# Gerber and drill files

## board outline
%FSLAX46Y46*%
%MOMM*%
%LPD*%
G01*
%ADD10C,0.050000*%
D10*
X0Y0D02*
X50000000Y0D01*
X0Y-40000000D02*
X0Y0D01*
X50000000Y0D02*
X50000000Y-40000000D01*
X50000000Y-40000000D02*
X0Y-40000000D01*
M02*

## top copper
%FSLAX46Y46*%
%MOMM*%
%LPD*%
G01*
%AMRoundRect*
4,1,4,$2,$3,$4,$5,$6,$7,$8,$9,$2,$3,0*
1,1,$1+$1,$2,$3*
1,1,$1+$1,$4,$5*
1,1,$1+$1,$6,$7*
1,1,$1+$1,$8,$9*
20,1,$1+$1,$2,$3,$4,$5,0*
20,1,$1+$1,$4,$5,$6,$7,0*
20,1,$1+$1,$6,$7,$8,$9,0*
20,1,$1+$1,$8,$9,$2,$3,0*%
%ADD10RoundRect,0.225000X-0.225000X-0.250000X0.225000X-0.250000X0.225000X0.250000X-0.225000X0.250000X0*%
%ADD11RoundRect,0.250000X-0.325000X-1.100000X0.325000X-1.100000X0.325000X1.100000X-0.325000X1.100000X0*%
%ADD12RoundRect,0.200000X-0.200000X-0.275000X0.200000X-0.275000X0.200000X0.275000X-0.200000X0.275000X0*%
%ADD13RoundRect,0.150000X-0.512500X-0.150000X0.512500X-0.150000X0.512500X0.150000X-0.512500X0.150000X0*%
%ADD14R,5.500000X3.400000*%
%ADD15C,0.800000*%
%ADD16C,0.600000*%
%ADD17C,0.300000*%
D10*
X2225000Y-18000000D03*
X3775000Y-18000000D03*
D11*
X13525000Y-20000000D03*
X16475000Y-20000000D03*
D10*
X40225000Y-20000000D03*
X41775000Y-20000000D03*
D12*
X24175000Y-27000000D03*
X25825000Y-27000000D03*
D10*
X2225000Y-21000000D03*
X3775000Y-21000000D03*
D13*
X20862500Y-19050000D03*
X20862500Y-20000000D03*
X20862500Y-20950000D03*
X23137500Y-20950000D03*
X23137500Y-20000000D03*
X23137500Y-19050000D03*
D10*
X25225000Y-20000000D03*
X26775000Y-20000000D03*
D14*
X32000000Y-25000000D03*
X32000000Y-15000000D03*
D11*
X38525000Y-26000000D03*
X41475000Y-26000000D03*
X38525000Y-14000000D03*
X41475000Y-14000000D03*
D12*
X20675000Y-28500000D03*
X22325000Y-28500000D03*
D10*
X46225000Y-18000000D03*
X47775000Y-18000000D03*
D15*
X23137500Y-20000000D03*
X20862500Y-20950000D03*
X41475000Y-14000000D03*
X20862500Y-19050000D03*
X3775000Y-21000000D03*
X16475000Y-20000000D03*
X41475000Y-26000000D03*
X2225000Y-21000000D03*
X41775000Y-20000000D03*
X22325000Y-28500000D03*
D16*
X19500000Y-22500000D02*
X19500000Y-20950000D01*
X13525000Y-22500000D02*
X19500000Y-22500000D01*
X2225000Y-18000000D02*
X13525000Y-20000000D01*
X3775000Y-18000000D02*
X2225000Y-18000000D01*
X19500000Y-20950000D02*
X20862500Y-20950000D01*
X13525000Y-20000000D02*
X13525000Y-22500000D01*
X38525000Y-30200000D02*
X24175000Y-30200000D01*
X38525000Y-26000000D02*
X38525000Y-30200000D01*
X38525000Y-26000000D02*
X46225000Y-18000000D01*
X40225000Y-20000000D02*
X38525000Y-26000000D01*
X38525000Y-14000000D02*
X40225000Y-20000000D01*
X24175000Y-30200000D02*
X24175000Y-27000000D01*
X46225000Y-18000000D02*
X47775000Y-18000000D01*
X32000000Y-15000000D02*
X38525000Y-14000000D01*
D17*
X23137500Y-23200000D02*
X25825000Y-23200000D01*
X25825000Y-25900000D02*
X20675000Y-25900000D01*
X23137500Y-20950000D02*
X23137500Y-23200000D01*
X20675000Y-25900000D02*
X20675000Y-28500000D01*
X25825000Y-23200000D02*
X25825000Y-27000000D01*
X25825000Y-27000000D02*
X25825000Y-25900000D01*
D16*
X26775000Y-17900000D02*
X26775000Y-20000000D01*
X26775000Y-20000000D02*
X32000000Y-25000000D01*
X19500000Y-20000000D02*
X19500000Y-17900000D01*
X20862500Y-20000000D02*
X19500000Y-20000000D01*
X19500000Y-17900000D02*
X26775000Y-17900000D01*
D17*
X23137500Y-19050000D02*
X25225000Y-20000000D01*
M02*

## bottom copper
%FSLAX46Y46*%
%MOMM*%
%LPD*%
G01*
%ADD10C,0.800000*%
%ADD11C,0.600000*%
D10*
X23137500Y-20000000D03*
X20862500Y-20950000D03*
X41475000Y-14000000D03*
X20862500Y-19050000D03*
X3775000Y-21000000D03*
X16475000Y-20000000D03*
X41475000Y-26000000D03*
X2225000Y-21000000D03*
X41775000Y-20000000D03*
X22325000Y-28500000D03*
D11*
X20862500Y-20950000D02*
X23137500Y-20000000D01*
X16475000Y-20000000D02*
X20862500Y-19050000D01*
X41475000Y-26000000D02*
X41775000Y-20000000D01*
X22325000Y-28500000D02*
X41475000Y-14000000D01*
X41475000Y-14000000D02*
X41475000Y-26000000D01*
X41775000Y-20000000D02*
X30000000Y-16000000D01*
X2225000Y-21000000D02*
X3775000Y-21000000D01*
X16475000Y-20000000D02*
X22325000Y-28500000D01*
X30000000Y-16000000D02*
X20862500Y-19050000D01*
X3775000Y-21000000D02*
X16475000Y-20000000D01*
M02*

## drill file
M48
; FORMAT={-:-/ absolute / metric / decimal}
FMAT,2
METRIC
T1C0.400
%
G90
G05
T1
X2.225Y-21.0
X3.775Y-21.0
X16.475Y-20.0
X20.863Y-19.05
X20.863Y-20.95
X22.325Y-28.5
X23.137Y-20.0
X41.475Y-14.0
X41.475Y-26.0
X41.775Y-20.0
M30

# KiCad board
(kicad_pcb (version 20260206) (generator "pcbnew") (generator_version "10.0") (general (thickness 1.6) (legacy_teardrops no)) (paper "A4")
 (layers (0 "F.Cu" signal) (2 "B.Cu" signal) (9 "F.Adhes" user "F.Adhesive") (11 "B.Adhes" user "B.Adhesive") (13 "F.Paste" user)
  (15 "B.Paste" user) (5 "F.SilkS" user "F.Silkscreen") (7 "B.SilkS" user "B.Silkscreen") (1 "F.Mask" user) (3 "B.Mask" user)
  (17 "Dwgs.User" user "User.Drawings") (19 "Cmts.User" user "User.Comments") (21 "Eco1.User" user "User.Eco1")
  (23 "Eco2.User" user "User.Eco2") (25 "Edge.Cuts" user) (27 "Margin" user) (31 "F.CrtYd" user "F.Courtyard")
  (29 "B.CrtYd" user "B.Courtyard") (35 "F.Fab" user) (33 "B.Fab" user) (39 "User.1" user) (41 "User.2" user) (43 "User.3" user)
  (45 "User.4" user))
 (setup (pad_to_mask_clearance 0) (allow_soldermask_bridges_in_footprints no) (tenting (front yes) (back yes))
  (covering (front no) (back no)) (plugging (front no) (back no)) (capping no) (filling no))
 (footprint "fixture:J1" (layer "F.Cu") (at 3 18)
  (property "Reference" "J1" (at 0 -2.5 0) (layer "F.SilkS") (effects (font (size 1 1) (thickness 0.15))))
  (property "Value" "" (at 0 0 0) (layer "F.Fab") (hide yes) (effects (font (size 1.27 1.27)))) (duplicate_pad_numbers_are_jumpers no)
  (pad "1" smd roundrect (at -0.775 0) (size 0.9 0.95) (layers "F.Cu" "F.Mask" "F.Paste") (roundrect_rratio 0.25) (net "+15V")
   (thermal_bridge_angle 45))
  (pad "2" smd roundrect (at 0.775 0) (size 0.9 0.95) (layers "F.Cu" "F.Mask" "F.Paste") (roundrect_rratio 0.25) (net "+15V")
   (thermal_bridge_angle 45)))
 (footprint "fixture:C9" (layer "F.Cu") (at 15 20)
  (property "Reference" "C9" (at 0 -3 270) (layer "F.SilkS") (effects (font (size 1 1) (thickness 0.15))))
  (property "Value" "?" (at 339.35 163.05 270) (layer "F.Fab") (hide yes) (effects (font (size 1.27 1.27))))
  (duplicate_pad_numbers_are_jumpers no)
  (pad "1" smd roundrect (at -1.475 0) (size 1.15 2.7) (layers "F.Cu" "F.Mask" "F.Paste") (roundrect_rratio 0.217391) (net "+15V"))
  (pad "2" smd roundrect (at 1.475 0) (size 1.15 2.7) (layers "F.Cu" "F.Mask" "F.Paste") (roundrect_rratio 0.217391) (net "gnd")))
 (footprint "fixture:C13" (layer "F.Cu") (at 41 20)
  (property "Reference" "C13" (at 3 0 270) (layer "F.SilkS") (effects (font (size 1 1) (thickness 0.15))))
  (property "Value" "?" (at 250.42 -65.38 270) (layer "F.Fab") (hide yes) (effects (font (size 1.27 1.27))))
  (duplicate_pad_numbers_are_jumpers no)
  (pad "1" smd roundrect (at -0.775 0) (size 0.9 0.95) (layers "F.Cu" "F.Mask" "F.Paste") (roundrect_rratio 0.25) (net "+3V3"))
  (pad "2" smd roundrect (at 0.775 0) (size 0.9 0.95) (layers "F.Cu" "F.Mask" "F.Paste") (roundrect_rratio 0.25) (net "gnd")))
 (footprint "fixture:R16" (layer "F.Cu") (at 25 27)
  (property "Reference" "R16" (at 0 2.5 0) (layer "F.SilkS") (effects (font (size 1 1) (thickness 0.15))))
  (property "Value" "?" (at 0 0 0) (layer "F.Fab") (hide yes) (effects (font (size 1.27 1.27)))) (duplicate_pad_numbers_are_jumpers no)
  (pad "1" smd roundrect (at -0.825 0) (size 0.8 0.95) (layers "F.Cu" "F.Mask" "F.Paste") (roundrect_rratio 0.25) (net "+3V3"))
  (pad "2" smd roundrect (at 0.825 0) (size 0.8 0.95) (layers "F.Cu" "F.Mask" "F.Paste") (roundrect_rratio 0.25) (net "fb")))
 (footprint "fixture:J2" (layer "F.Cu") (at 3 21)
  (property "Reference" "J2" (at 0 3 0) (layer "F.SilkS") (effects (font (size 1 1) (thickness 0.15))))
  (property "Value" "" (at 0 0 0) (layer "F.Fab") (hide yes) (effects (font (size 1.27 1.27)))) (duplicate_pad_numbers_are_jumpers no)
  (pad "1" smd roundrect (at -0.775 0) (size 0.9 0.95) (layers "F.Cu" "F.Mask" "F.Paste") (roundrect_rratio 0.25) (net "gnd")
   (thermal_bridge_angle 45))
  (pad "2" smd roundrect (at 0.775 0) (size 0.9 0.95) (layers "F.Cu" "F.Mask" "F.Paste") (roundrect_rratio 0.25) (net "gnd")
   (thermal_bridge_angle 45)))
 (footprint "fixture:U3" (layer "F.Cu") (at 22 20)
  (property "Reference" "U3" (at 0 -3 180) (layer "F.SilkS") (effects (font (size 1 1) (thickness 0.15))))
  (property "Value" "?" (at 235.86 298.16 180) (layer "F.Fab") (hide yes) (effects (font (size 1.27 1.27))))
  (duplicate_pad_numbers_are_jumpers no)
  (pad "1" smd roundrect (at -1.1375 -0.95) (size 1.325 0.6) (layers "F.Cu" "F.Mask" "F.Paste") (roundrect_rratio 0.25) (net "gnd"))
  (pad "2" smd roundrect (at -1.1375 0) (size 1.325 0.6) (layers "F.Cu" "F.Mask" "F.Paste") (roundrect_rratio 0.25) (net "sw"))
  (pad "3" smd roundrect (at -1.1375 0.95) (size 1.325 0.6) (layers "F.Cu" "F.Mask" "F.Paste") (roundrect_rratio 0.25) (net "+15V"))
  (pad "4" smd roundrect (at 1.1375 0.95) (size 1.325 0.6) (layers "F.Cu" "F.Mask" "F.Paste") (roundrect_rratio 0.25) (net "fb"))
  (pad "5" smd roundrect (at 1.1375 0) (size 1.325 0.6) (layers "F.Cu" "F.Mask" "F.Paste") (roundrect_rratio 0.25) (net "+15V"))
  (pad "6" smd roundrect (at 1.1375 -0.95) (size 1.325 0.6) (layers "F.Cu" "F.Mask" "F.Paste") (roundrect_rratio 0.25) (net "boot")))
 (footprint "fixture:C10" (layer "F.Cu") (at 26 20)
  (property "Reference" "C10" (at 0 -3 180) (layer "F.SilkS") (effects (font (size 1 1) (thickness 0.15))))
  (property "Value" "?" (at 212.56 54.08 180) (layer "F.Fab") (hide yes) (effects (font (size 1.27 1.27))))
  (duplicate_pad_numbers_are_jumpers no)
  (pad "1" smd roundrect (at -0.775 0) (size 0.9 0.95) (layers "F.Cu" "F.Mask" "F.Paste") (roundrect_rratio 0.25) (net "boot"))
  (pad "2" smd roundrect (at 0.775 0) (size 0.9 0.95) (layers "F.Cu" "F.Mask" "F.Paste") (roundrect_rratio 0.25) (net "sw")))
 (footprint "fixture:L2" (layer "F.Cu") (at 32 20 90)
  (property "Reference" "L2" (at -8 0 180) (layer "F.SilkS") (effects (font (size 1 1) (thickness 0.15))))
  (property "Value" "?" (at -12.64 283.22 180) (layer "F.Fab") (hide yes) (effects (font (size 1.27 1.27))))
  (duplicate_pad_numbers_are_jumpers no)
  (pad "1" smd rect (at -5 0 90) (size 3.4 5.5) (layers "F.Cu" "F.Mask" "F.Paste") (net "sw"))
  (pad "2" smd rect (at 5 0 90) (size 3.4 5.5) (layers "F.Cu" "F.Mask" "F.Paste") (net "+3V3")))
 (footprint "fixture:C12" (layer "F.Cu") (at 40 26)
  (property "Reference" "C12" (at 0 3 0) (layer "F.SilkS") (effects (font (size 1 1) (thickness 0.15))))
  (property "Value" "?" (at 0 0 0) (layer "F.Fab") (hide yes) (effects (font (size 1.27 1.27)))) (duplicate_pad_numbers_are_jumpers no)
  (pad "1" smd roundrect (at -1.475 0) (size 1.15 2.7) (layers "F.Cu" "F.Mask" "F.Paste") (roundrect_rratio 0.217391) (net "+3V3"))
  (pad "2" smd roundrect (at 1.475 0) (size 1.15 2.7) (layers "F.Cu" "F.Mask" "F.Paste") (roundrect_rratio 0.217391) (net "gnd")))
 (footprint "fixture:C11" (layer "F.Cu") (at 40 14)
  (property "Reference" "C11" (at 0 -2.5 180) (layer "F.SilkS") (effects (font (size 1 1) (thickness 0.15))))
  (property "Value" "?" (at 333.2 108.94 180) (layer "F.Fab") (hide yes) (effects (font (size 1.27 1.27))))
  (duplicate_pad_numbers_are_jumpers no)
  (pad "1" smd roundrect (at -1.475 0) (size 1.15 2.7) (layers "F.Cu" "F.Mask" "F.Paste") (roundrect_rratio 0.217391) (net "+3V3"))
  (pad "2" smd roundrect (at 1.475 0) (size 1.15 2.7) (layers "F.Cu" "F.Mask" "F.Paste") (roundrect_rratio 0.217391) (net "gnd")))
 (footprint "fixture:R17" (layer "F.Cu") (at 21.5 28.5)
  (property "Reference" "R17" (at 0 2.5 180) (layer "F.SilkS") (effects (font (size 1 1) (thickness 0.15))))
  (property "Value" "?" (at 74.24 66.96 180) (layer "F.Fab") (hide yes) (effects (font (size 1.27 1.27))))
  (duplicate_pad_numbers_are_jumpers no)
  (pad "1" smd roundrect (at -0.825 0) (size 0.8 0.95) (layers "F.Cu" "F.Mask" "F.Paste") (roundrect_rratio 0.25) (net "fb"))
  (pad "2" smd roundrect (at 0.825 0) (size 0.8 0.95) (layers "F.Cu" "F.Mask" "F.Paste") (roundrect_rratio 0.25) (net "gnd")))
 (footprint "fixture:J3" (layer "F.Cu") (at 47 18)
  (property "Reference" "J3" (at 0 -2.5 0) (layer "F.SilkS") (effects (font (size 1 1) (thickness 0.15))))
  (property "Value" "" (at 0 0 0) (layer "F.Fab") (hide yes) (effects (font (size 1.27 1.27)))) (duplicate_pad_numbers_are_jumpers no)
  (pad "1" smd roundrect (at -0.775 0) (size 0.9 0.95) (layers "F.Cu" "F.Mask" "F.Paste") (roundrect_rratio 0.25) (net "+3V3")
   (thermal_bridge_angle 45))
  (pad "2" smd roundrect (at 0.775 0) (size 0.9 0.95) (layers "F.Cu" "F.Mask" "F.Paste") (roundrect_rratio 0.25) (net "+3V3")
   (thermal_bridge_angle 45)))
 (gr_line (start 0 0) (end 50 0) (stroke (width 0.05) (type default)) (layer "Edge.Cuts"))
 (gr_line (start 0 40) (end 0 0) (stroke (width 0.05) (type default)) (layer "Edge.Cuts"))
 (gr_line (start 50 0) (end 50 40) (stroke (width 0.05) (type default)) (layer "Edge.Cuts"))
 (gr_line (start 50 40) (end 0 40) (stroke (width 0.05) (type default)) (layer "Edge.Cuts"))
 (segment (start 19.5 22.5) (end 19.5 20.95) (width 0.6) (layer "F.Cu") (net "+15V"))
 (segment (start 13.525 22.5) (end 19.5 22.5) (width 0.6) (layer "F.Cu") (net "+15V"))
 (segment (start 2.225 18) (end 13.525 20) (width 0.6) (layer "F.Cu") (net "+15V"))
 (segment (start 3.775 18) (end 2.225 18) (width 0.6) (layer "F.Cu") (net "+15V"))
 (segment (start 19.5 20.95) (end 20.8625 20.95) (width 0.6) (layer "F.Cu") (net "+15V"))
 (segment (start 13.525 20) (end 13.525 22.5) (width 0.6) (layer "F.Cu") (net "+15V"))
 (via (at 23.1375 20) (size 0.8) (drill 0.4) (layers "F.Cu" "B.Cu") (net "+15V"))
 (via (at 20.8625 20.95) (size 0.8) (drill 0.4) (layers "F.Cu" "B.Cu") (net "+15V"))
 (segment (start 20.8625 20.95) (end 23.1375 20) (width 0.6) (layer "B.Cu") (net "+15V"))
 (via (at 41.475 14) (size 0.8) (drill 0.4) (layers "F.Cu" "B.Cu") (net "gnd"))
 (via (at 20.8625 19.05) (size 0.8) (drill 0.4) (layers "F.Cu" "B.Cu") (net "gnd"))
 (via (at 3.775 21) (size 0.8) (drill 0.4) (layers "F.Cu" "B.Cu") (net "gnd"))
 (via (at 16.475 20) (size 0.8) (drill 0.4) (layers "F.Cu" "B.Cu") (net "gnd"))
 (via (at 41.475 26) (size 0.8) (drill 0.4) (layers "F.Cu" "B.Cu") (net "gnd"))
 (via (at 2.225 21) (size 0.8) (drill 0.4) (layers "F.Cu" "B.Cu") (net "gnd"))
 (via (at 41.775 20) (size 0.8) (drill 0.4) (layers "F.Cu" "B.Cu") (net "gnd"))
 (via (at 22.325 28.5) (size 0.8) (drill 0.4) (layers "F.Cu" "B.Cu") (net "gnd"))
 (segment (start 16.475 20) (end 20.8625 19.05) (width 0.6) (layer "B.Cu") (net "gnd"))
 (segment (start 41.475 26) (end 41.775 20) (width 0.6) (layer "B.Cu") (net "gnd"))
 (segment (start 22.325 28.5) (end 41.475 14) (width 0.6) (layer "B.Cu") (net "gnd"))
 (segment (start 41.475 14) (end 41.475 26) (width 0.6) (layer "B.Cu") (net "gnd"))
 (segment (start 41.775 20) (end 30 16) (width 0.6) (layer "B.Cu") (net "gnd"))
 (segment (start 2.225 21) (end 3.775 21) (width 0.6) (layer "B.Cu") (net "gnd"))
 (segment (start 16.475 20) (end 22.325 28.5) (width 0.6) (layer "B.Cu") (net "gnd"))
 (segment (start 30 16) (end 20.8625 19.05) (width 0.6) (layer "B.Cu") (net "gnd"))
 (segment (start 3.775 21) (end 16.475 20) (width 0.6) (layer "B.Cu") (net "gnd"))
 (segment (start 38.525 30.2) (end 24.175 30.2) (width 0.6) (layer "F.Cu") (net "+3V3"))
 (segment (start 38.525 26) (end 38.525 30.2) (width 0.6) (layer "F.Cu") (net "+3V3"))
 (segment (start 38.525 26) (end 46.225 18) (width 0.6) (layer "F.Cu") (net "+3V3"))
 (segment (start 40.225 20) (end 38.525 26) (width 0.6) (layer "F.Cu") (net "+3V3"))
 (segment (start 38.525 14) (end 40.225 20) (width 0.6) (layer "F.Cu") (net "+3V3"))
 (segment (start 24.175 30.2) (end 24.175 27) (width 0.6) (layer "F.Cu") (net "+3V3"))
 (segment (start 46.225 18) (end 47.775 18) (width 0.6) (layer "F.Cu") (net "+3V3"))
 (segment (start 32 15) (end 38.525 14) (width 0.6) (layer "F.Cu") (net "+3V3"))
 (segment (start 23.1375 23.2) (end 25.825 23.2) (width 0.3) (layer "F.Cu") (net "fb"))
 (segment (start 25.825 25.9) (end 20.675 25.9) (width 0.3) (layer "F.Cu") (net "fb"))
 (segment (start 23.1375 20.95) (end 23.1375 23.2) (width 0.3) (layer "F.Cu") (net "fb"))
 (segment (start 20.675 25.9) (end 20.675 28.5) (width 0.3) (layer "F.Cu") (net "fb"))
 (segment (start 25.825 23.2) (end 25.825 27) (width 0.3) (layer "F.Cu") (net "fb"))
 (segment (start 25.825 27) (end 25.825 25.9) (width 0.3) (layer "F.Cu") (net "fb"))
 (segment (start 26.775 17.9) (end 26.775 20) (width 0.6) (layer "F.Cu") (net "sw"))
 (segment (start 26.775 20) (end 32 25) (width 0.6) (layer "F.Cu") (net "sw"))
 (segment (start 19.5 20) (end 19.5 17.9) (width 0.6) (layer "F.Cu") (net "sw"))
 (segment (start 20.8625 20) (end 19.5 20) (width 0.6) (layer "F.Cu") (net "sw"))
 (segment (start 19.5 17.9) (end 26.775 17.9) (width 0.6) (layer "F.Cu") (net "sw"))
 (segment (start 23.1375 19.05) (end 25.225 20) (width 0.3) (layer "F.Cu") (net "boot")))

